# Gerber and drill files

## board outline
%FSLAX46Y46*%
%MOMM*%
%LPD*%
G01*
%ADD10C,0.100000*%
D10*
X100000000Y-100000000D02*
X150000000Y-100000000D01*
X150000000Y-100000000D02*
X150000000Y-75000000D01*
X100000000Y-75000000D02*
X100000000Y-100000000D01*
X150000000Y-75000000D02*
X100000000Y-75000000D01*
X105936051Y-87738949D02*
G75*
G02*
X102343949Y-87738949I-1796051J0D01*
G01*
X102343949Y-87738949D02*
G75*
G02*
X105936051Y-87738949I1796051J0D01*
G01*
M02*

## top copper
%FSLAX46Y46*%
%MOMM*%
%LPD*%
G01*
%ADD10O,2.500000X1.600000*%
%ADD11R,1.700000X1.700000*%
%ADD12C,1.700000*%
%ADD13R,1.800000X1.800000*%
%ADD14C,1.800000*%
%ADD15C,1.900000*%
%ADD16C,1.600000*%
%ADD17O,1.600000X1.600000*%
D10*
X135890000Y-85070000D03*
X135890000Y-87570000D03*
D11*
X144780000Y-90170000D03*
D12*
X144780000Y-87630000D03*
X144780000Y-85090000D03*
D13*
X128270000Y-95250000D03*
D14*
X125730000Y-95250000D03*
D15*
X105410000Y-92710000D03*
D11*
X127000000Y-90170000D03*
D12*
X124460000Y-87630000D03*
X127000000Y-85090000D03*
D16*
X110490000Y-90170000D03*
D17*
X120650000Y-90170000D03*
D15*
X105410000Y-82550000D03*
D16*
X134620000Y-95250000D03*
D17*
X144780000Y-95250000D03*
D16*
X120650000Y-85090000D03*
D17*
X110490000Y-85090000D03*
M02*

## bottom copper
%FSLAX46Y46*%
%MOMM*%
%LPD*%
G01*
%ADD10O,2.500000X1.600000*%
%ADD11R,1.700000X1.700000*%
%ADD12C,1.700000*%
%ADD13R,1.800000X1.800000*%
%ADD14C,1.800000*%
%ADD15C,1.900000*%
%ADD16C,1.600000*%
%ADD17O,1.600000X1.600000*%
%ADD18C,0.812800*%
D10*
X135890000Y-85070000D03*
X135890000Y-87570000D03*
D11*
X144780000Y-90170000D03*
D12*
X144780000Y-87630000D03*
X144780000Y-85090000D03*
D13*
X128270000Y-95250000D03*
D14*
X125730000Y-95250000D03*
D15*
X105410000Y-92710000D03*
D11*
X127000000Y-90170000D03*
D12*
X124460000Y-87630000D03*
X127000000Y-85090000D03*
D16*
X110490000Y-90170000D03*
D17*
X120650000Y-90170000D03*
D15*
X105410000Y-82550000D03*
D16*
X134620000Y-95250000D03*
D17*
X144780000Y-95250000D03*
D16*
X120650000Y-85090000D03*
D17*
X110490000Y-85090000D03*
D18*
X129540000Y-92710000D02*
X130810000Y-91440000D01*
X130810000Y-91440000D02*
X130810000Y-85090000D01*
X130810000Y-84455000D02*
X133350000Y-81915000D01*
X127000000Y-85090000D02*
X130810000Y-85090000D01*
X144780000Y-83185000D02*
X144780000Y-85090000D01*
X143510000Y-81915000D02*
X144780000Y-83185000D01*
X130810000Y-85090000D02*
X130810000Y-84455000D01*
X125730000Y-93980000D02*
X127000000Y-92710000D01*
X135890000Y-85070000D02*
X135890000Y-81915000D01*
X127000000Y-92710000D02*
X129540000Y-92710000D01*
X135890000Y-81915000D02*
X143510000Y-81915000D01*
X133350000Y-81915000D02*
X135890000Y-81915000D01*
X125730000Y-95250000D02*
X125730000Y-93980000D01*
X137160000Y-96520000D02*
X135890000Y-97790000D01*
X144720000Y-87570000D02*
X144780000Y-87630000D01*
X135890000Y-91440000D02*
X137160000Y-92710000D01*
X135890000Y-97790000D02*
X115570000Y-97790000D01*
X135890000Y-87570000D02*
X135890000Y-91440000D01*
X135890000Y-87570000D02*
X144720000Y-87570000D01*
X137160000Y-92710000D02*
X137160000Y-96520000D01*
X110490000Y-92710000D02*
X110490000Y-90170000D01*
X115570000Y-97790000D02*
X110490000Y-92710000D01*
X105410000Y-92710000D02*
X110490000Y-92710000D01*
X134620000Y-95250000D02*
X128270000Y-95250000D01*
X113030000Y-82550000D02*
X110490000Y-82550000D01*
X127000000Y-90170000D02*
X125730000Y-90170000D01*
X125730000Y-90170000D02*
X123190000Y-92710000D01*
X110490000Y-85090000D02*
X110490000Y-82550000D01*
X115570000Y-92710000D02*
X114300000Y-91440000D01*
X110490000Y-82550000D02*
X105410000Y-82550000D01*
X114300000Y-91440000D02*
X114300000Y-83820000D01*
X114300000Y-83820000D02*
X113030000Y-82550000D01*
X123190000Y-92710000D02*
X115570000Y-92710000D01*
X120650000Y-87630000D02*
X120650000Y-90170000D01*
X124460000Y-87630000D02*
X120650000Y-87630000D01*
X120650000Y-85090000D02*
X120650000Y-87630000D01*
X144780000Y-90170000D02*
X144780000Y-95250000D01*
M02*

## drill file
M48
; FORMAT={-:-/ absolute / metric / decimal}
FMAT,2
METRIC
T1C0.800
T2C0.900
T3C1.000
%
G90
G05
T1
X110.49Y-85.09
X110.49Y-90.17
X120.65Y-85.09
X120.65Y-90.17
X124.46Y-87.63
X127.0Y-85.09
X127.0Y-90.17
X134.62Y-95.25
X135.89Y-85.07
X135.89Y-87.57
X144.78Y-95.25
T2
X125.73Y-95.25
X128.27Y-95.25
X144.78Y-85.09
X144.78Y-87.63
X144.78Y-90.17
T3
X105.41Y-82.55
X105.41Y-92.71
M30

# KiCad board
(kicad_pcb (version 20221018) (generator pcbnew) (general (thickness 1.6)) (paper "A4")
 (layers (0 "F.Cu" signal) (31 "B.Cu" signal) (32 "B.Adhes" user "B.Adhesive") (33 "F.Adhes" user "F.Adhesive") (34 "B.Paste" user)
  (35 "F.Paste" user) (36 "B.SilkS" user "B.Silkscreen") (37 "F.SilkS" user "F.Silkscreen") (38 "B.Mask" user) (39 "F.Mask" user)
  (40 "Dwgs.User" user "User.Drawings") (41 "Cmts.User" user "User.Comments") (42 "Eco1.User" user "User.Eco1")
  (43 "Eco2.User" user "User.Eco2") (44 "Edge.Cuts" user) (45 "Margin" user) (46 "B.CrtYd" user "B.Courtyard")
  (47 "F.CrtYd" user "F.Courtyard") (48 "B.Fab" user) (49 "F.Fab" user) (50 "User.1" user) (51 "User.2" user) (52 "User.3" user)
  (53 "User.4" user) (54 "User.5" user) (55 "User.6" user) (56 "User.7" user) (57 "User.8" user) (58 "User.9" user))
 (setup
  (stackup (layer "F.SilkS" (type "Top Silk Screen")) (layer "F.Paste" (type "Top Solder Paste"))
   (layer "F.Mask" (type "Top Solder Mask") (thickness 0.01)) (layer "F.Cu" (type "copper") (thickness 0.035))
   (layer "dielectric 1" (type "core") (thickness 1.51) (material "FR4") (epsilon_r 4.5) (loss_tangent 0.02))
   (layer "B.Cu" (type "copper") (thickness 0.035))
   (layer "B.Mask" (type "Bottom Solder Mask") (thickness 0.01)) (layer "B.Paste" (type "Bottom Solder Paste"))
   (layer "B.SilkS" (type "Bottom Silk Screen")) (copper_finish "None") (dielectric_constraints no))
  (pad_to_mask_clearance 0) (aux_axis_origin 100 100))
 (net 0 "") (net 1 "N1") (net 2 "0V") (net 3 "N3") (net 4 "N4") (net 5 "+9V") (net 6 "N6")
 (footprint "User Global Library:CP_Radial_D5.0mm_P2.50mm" (layer "F.Cu") (at 135.89 86.32 -90)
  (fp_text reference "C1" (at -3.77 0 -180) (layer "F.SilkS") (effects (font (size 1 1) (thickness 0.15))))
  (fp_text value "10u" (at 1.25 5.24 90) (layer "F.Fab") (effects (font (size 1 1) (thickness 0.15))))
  (pad "1" thru_hole oval (at -1.25 0 270) (size 1.6 2.5) (drill 0.8) (layers "*.Cu" "*.Mask") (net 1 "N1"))
  (pad "2" thru_hole oval (at 1.25 0 270) (size 1.6 2.5) (drill 0.8) (layers "*.Cu" "*.Mask") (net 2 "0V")))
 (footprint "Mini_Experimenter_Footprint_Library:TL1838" (layer "F.Cu") (at 144.78 87.63 90)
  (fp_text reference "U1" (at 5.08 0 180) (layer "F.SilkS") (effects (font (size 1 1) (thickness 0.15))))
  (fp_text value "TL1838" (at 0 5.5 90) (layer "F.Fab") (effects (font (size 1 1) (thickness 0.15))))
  (pad "1" thru_hole rect (at -2.54 0 90) (size 1.7 1.7) (drill 0.9) (layers "*.Cu" "*.Mask") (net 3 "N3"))
  (pad "2" thru_hole circle (at 0 0 90) (size 1.7 1.7) (drill 0.9) (layers "*.Cu" "*.Mask") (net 2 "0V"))
  (pad "3" thru_hole circle (at 2.54 0 90) (size 1.7 1.7) (drill 0.9) (layers "*.Cu" "*.Mask") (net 1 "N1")))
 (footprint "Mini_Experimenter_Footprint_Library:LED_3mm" (layer "F.Cu") (at 128.27 95.25 180)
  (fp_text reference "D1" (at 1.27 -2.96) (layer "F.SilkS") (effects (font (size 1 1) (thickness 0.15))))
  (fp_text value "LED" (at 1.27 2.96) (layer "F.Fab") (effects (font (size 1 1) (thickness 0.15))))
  (pad "1" thru_hole rect (at 0 0 180) (size 1.8 1.8) (drill 0.9) (layers "*.Cu" "*.Mask") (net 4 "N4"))
  (pad "2" thru_hole circle (at 2.54 0 180) (size 1.8 1.8) (drill 0.9) (layers "*.Cu" "*.Mask") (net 1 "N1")))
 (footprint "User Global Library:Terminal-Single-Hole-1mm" (layer "F.Cu") (at 105.41 92.71)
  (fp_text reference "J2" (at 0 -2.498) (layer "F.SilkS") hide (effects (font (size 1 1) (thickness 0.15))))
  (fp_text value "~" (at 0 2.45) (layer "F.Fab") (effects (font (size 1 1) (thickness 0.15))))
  (pad "1" thru_hole circle (at 0 0) (size 1.9 1.9) (drill 1) (layers "*.Cu" "*.Mask") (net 2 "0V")))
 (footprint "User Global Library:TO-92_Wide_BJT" (layer "F.Cu") (at 127 90.17 90)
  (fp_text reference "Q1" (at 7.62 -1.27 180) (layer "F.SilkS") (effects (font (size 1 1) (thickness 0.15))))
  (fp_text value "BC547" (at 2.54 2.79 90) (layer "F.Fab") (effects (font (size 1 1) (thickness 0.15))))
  (pad "1" thru_hole rect (at 0 0 90) (size 1.7 1.7) (drill 0.8) (layers "*.Cu" "*.Mask") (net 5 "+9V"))
  (pad "2" thru_hole circle (at 2.54 -2.54 90) (size 1.7 1.7) (drill 0.8) (layers "*.Cu" "*.Mask") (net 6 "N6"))
  (pad "3" thru_hole circle (at 5.08 0 90) (size 1.7 1.7) (drill 0.8) (layers "*.Cu" "*.Mask") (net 1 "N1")))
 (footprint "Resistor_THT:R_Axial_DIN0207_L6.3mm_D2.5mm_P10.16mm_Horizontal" (layer "F.Cu") (at 110.49 90.17)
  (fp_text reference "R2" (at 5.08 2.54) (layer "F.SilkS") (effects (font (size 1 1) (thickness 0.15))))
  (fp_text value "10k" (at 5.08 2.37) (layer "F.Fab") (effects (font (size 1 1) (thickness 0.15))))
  (pad "1" thru_hole circle (at 0 0) (size 1.6 1.6) (drill 0.8) (layers "*.Cu" "*.Mask") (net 2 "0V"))
  (pad "2" thru_hole oval (at 10.16 0) (size 1.6 1.6) (drill 0.8) (layers "*.Cu" "*.Mask") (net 6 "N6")))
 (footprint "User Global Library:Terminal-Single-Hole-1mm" (layer "F.Cu") (at 105.41 82.55)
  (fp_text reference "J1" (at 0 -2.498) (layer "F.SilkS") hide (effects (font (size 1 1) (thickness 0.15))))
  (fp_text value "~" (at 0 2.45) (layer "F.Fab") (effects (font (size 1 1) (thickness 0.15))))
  (pad "1" thru_hole circle (at 0 0) (size 1.9 1.9) (drill 1) (layers "*.Cu" "*.Mask") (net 5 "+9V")))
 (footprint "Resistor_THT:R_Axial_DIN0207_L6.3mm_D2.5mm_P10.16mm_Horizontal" (layer "F.Cu") (at 134.62 95.25)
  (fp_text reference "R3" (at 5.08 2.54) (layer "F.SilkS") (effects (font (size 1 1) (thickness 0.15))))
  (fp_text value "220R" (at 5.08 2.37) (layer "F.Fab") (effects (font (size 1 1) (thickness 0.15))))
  (pad "1" thru_hole circle (at 0 0) (size 1.6 1.6) (drill 0.8) (layers "*.Cu" "*.Mask") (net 4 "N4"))
  (pad "2" thru_hole oval (at 10.16 0) (size 1.6 1.6) (drill 0.8) (layers "*.Cu" "*.Mask") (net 3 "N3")))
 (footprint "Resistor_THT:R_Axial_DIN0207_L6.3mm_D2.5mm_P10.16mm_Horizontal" (layer "F.Cu") (at 120.65 85.09 180)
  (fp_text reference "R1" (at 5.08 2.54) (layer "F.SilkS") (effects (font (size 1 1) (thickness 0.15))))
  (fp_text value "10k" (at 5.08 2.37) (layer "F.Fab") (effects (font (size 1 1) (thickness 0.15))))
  (pad "1" thru_hole circle (at 0 0 180) (size 1.6 1.6) (drill 0.8) (layers "*.Cu" "*.Mask") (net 6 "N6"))
  (pad "2" thru_hole oval (at 10.16 0 180) (size 1.6 1.6) (drill 0.8) (layers "*.Cu" "*.Mask") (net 5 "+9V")))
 (gr_line (start 100 100) (end 150 100) (stroke (width 0.1) (type default)) (layer "Edge.Cuts"))
 (gr_line (start 150 100) (end 150 75) (stroke (width 0.1) (type default)) (layer "Edge.Cuts"))
 (gr_line (start 100 75) (end 100 100) (stroke (width 0.1) (type default)) (layer "Edge.Cuts"))
 (gr_line (start 150 75) (end 100 75) (stroke (width 0.1) (type default)) (layer "Edge.Cuts"))
 (gr_circle (center 104.14 87.738949) (end 105.41 89.008949) (stroke (width 0.1) (type default)) (fill none) (layer "Edge.Cuts"))
 (segment (start 129.54 92.71) (end 130.81 91.44) (width 0.8128) (layer "B.Cu") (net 1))
 (segment (start 130.81 91.44) (end 130.81 85.09) (width 0.8128) (layer "B.Cu") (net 1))
 (segment (start 130.81 84.455) (end 133.35 81.915) (width 0.8128) (layer "B.Cu") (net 1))
 (segment (start 127 85.09) (end 130.81 85.09) (width 0.8128) (layer "B.Cu") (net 1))
 (segment (start 144.78 83.185) (end 144.78 85.09) (width 0.8128) (layer "B.Cu") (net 1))
 (segment (start 143.51 81.915) (end 144.78 83.185) (width 0.8128) (layer "B.Cu") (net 1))
 (segment (start 130.81 85.09) (end 130.81 84.455) (width 0.8128) (layer "B.Cu") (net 1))
 (segment (start 125.73 93.98) (end 127 92.71) (width 0.8128) (layer "B.Cu") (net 1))
 (segment (start 135.89 85.07) (end 135.89 81.915) (width 0.8128) (layer "B.Cu") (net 1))
 (segment (start 127 92.71) (end 129.54 92.71) (width 0.8128) (layer "B.Cu") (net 1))
 (segment (start 135.89 81.915) (end 143.51 81.915) (width 0.8128) (layer "B.Cu") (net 1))
 (segment (start 133.35 81.915) (end 135.89 81.915) (width 0.8128) (layer "B.Cu") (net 1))
 (segment (start 125.73 95.25) (end 125.73 93.98) (width 0.8128) (layer "B.Cu") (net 1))
 (segment (start 137.16 96.52) (end 135.89 97.79) (width 0.8128) (layer "B.Cu") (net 2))
 (segment (start 144.72 87.57) (end 144.78 87.63) (width 0.8128) (layer "B.Cu") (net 2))
 (segment (start 135.89 91.44) (end 137.16 92.71) (width 0.8128) (layer "B.Cu") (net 2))
 (segment (start 135.89 97.79) (end 115.57 97.79) (width 0.8128) (layer "B.Cu") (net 2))
 (segment (start 135.89 87.57) (end 135.89 91.44) (width 0.8128) (layer "B.Cu") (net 2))
 (segment (start 135.89 87.57) (end 144.72 87.57) (width 0.8128) (layer "B.Cu") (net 2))
 (segment (start 137.16 92.71) (end 137.16 96.52) (width 0.8128) (layer "B.Cu") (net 2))
 (segment (start 110.49 92.71) (end 110.49 90.17) (width 0.8128) (layer "B.Cu") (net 2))
 (segment (start 115.57 97.79) (end 110.49 92.71) (width 0.8128) (layer "B.Cu") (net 2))
 (segment (start 105.41 92.71) (end 110.49 92.71) (width 0.8128) (layer "B.Cu") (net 2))
 (segment (start 134.62 95.25) (end 128.27 95.25) (width 0.8128) (layer "B.Cu") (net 4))
 (segment (start 113.03 82.55) (end 110.49 82.55) (width 0.8128) (layer "B.Cu") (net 5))
 (segment (start 127 90.17) (end 125.73 90.17) (width 0.8128) (layer "B.Cu") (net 5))
 (segment (start 125.73 90.17) (end 123.19 92.71) (width 0.8128) (layer "B.Cu") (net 5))
 (segment (start 110.49 85.09) (end 110.49 82.55) (width 0.8128) (layer "B.Cu") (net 5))
 (segment (start 115.57 92.71) (end 114.3 91.44) (width 0.8128) (layer "B.Cu") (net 5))
 (segment (start 110.49 82.55) (end 105.41 82.55) (width 0.8128) (layer "B.Cu") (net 5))
 (segment (start 114.3 91.44) (end 114.3 83.82) (width 0.8128) (layer "B.Cu") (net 5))
 (segment (start 114.3 83.82) (end 113.03 82.55) (width 0.8128) (layer "B.Cu") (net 5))
 (segment (start 123.19 92.71) (end 115.57 92.71) (width 0.8128) (layer "B.Cu") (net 5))
 (segment (start 120.65 87.63) (end 120.65 90.17) (width 0.8128) (layer "B.Cu") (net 6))
 (segment (start 124.46 87.63) (end 120.65 87.63) (width 0.8128) (layer "B.Cu") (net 6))
 (segment (start 120.65 85.09) (end 120.65 87.63) (width 0.8128) (layer "B.Cu") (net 6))
 (segment (start 144.78 90.17) (end 144.78 95.25) (width 0.8128) (layer "B.Cu") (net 3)))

